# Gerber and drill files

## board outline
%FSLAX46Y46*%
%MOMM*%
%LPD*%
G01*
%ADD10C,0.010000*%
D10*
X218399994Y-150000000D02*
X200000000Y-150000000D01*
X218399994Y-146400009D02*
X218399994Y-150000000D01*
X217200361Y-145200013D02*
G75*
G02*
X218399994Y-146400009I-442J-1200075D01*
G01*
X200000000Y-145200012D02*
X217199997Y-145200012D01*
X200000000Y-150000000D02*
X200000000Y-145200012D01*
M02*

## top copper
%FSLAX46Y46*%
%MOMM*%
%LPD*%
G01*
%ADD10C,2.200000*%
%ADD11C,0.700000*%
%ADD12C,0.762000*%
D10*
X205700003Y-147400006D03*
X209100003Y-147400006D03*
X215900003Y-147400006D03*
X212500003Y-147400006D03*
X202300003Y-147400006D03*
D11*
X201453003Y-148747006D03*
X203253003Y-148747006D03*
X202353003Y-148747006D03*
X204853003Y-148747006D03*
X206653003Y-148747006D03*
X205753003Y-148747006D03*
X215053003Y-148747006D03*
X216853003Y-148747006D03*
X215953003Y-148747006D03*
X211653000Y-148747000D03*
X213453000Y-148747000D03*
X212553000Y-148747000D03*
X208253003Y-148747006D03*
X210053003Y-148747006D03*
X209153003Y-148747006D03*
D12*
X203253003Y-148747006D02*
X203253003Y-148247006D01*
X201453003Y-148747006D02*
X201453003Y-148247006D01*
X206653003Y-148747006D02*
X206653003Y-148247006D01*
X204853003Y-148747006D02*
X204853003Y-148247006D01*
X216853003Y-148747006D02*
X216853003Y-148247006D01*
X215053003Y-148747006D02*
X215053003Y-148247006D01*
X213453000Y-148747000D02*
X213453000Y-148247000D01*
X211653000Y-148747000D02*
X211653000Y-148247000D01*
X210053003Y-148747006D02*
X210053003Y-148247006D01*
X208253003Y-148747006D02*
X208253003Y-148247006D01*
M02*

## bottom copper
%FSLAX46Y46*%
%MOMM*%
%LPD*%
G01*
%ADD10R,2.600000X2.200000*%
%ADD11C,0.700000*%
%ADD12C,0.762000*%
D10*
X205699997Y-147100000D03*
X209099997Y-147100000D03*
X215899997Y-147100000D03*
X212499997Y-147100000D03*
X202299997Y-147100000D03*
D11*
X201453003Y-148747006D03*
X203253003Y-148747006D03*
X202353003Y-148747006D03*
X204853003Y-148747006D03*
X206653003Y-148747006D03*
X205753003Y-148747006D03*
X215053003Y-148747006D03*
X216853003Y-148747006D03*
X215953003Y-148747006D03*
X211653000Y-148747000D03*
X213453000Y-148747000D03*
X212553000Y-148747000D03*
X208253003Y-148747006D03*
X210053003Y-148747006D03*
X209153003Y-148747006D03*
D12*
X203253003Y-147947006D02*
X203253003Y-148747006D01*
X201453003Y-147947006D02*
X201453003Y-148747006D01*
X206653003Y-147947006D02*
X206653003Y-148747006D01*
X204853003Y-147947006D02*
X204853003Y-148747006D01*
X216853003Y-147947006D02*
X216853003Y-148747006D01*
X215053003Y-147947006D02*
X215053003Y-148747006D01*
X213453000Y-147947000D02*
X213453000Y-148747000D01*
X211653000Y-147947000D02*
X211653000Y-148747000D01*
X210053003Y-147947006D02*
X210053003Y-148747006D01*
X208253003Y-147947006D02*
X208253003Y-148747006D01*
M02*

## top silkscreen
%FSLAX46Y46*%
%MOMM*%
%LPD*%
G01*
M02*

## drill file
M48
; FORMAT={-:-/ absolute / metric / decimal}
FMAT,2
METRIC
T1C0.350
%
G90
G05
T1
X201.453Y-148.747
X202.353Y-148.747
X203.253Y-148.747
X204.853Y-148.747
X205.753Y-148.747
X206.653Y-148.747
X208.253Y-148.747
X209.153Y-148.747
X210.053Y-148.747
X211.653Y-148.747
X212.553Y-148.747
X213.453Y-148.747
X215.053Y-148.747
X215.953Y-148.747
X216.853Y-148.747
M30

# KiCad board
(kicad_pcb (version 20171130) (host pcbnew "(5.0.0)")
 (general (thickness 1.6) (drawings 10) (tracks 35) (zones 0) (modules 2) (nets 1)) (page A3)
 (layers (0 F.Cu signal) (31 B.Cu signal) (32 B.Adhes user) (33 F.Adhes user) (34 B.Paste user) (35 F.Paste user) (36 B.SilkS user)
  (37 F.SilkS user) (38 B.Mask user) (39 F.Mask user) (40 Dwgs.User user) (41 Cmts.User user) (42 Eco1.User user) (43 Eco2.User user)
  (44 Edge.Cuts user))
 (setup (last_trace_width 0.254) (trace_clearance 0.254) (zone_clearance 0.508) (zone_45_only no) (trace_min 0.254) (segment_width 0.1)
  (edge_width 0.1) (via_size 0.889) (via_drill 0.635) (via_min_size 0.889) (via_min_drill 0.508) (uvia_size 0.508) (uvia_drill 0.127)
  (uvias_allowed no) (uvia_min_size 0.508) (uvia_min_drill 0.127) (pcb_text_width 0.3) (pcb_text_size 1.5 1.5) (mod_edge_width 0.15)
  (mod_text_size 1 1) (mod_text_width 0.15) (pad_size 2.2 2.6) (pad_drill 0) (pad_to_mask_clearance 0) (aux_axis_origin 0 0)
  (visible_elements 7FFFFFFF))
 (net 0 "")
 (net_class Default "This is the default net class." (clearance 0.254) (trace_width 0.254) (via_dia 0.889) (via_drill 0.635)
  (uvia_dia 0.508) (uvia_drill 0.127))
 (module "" (layer B.Cu) (at 215.800003 147.500006 270)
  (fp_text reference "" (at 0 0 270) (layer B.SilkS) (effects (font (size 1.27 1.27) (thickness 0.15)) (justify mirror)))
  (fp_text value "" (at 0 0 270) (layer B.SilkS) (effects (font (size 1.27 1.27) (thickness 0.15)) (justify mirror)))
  (pad 2 smd circle (at -0.1 10.1 270) (size 2.2 2.2) (layers F.Cu F.Mask))
  (pad 3 smd circle (at -0.1 6.7 270) (size 2.2 2.2) (layers F.Cu F.Mask))
  (pad 5 smd circle (at -0.1 -0.1 270) (size 2.2 2.2) (layers F.Cu F.Mask))
  (pad 4 smd circle (at -0.1 3.3 270) (size 2.2 2.2) (layers F.Cu F.Mask))
  (pad 1 smd circle (at -0.1 13.5 270) (size 2.2 2.2) (layers F.Cu F.Mask)))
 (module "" (layer F.Cu) (at 215.799997 147.800006 90)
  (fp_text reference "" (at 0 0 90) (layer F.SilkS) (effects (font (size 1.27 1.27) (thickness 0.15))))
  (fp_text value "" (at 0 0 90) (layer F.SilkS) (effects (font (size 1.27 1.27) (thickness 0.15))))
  (pad 2 smd rect (at 0.700006 -10.1 90) (size 2.2 2.6) (layers B.Cu B.Mask))
  (pad 3 smd rect (at 0.700006 -6.7 90) (size 2.2 2.6) (layers B.Cu B.Mask))
  (pad 5 smd rect (at 0.700006 0.1 90) (size 2.2 2.6) (layers B.Cu B.Mask))
  (pad 4 smd rect (at 0.700006 -3.3 90) (size 2.2 2.6) (layers B.Cu B.Mask))
  (pad 1 smd rect (at 0.700006 -13.5 90) (size 2.2 2.6) (layers B.Cu B.Mask)))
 (gr_line (start 218.399994 150) (end 200 150) (angle 90) (layer Edge.Cuts) (width 0.01))
 (gr_line (start 218.399994 146.400009) (end 218.399994 150) (angle 90) (layer Edge.Cuts) (width 0.01))
 (gr_arc (start 217.199919 146.400088) (end 218.399994 146.400009) (angle -89.97513145) (layer Edge.Cuts) (width 0.01))
 (gr_line (start 200 145.200012) (end 217.199997 145.200012) (angle 90) (layer Edge.Cuts) (width 0.01))
 (gr_line (start 200 150) (end 200 145.200012) (angle 90) (layer Edge.Cuts) (width 0.01))
 (via (at 201.453003 148.747006) (size 0.7) (drill 0.35) (layers F.Cu B.Cu) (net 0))
 (via (at 203.253003 148.747006) (size 0.7) (drill 0.35) (layers F.Cu B.Cu) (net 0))
 (via (at 202.353003 148.747006) (size 0.7) (drill 0.35) (layers F.Cu B.Cu) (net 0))
 (segment (start 203.253003 147.947006) (end 203.253003 148.747006) (width 0.762) (layer B.Cu) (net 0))
 (segment (start 203.253003 148.747006) (end 203.253003 148.247006) (width 0.762) (layer F.Cu) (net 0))
 (segment (start 201.453003 147.947006) (end 201.453003 148.747006) (width 0.762) (layer B.Cu) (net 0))
 (segment (start 201.453003 148.747006) (end 201.453003 148.247006) (width 0.762) (layer F.Cu) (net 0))
 (via (at 204.853003 148.747006) (size 0.7) (drill 0.35) (layers F.Cu B.Cu) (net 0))
 (via (at 206.653003 148.747006) (size 0.7) (drill 0.35) (layers F.Cu B.Cu) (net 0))
 (via (at 205.753003 148.747006) (size 0.7) (drill 0.35) (layers F.Cu B.Cu) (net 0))
 (segment (start 206.653003 147.947006) (end 206.653003 148.747006) (width 0.762) (layer B.Cu) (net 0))
 (segment (start 206.653003 148.747006) (end 206.653003 148.247006) (width 0.762) (layer F.Cu) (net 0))
 (segment (start 204.853003 147.947006) (end 204.853003 148.747006) (width 0.762) (layer B.Cu) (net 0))
 (segment (start 204.853003 148.747006) (end 204.853003 148.247006) (width 0.762) (layer F.Cu) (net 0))
 (via (at 215.053003 148.747006) (size 0.7) (drill 0.35) (layers F.Cu B.Cu) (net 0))
 (via (at 216.853003 148.747006) (size 0.7) (drill 0.35) (layers F.Cu B.Cu) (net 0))
 (via (at 215.953003 148.747006) (size 0.7) (drill 0.35) (layers F.Cu B.Cu) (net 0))
 (segment (start 216.853003 147.947006) (end 216.853003 148.747006) (width 0.762) (layer B.Cu) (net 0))
 (segment (start 216.853003 148.747006) (end 216.853003 148.247006) (width 0.762) (layer F.Cu) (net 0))
 (segment (start 215.053003 147.947006) (end 215.053003 148.747006) (width 0.762) (layer B.Cu) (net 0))
 (segment (start 215.053003 148.747006) (end 215.053003 148.247006) (width 0.762) (layer F.Cu) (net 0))
 (via (at 211.653 148.747) (size 0.7) (drill 0.35) (layers F.Cu B.Cu) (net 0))
 (via (at 213.453 148.747) (size 0.7) (drill 0.35) (layers F.Cu B.Cu) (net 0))
 (via (at 212.553 148.747) (size 0.7) (drill 0.35) (layers F.Cu B.Cu) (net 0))
 (segment (start 213.453 147.947) (end 213.453 148.747) (width 0.762) (layer B.Cu) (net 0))
 (segment (start 213.453 148.747) (end 213.453 148.247) (width 0.762) (layer F.Cu) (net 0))
 (segment (start 211.653 147.947) (end 211.653 148.747) (width 0.762) (layer B.Cu) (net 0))
 (segment (start 211.653 148.747) (end 211.653 148.247) (width 0.762) (layer F.Cu) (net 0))
 (via (at 208.253003 148.747006) (size 0.7) (drill 0.35) (layers F.Cu B.Cu) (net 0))
 (via (at 210.053003 148.747006) (size 0.7) (drill 0.35) (layers F.Cu B.Cu) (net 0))
 (via (at 209.153003 148.747006) (size 0.7) (drill 0.35) (layers F.Cu B.Cu) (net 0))
 (segment (start 210.053003 147.947006) (end 210.053003 148.747006) (width 0.762) (layer B.Cu) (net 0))
 (segment (start 210.053003 148.747006) (end 210.053003 148.247006) (width 0.762) (layer F.Cu) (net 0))
 (segment (start 208.253003 147.947006) (end 208.253003 148.747006) (width 0.762) (layer B.Cu) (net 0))
 (segment (start 208.253003 148.747006) (end 208.253003 148.247006) (width 0.762) (layer F.Cu) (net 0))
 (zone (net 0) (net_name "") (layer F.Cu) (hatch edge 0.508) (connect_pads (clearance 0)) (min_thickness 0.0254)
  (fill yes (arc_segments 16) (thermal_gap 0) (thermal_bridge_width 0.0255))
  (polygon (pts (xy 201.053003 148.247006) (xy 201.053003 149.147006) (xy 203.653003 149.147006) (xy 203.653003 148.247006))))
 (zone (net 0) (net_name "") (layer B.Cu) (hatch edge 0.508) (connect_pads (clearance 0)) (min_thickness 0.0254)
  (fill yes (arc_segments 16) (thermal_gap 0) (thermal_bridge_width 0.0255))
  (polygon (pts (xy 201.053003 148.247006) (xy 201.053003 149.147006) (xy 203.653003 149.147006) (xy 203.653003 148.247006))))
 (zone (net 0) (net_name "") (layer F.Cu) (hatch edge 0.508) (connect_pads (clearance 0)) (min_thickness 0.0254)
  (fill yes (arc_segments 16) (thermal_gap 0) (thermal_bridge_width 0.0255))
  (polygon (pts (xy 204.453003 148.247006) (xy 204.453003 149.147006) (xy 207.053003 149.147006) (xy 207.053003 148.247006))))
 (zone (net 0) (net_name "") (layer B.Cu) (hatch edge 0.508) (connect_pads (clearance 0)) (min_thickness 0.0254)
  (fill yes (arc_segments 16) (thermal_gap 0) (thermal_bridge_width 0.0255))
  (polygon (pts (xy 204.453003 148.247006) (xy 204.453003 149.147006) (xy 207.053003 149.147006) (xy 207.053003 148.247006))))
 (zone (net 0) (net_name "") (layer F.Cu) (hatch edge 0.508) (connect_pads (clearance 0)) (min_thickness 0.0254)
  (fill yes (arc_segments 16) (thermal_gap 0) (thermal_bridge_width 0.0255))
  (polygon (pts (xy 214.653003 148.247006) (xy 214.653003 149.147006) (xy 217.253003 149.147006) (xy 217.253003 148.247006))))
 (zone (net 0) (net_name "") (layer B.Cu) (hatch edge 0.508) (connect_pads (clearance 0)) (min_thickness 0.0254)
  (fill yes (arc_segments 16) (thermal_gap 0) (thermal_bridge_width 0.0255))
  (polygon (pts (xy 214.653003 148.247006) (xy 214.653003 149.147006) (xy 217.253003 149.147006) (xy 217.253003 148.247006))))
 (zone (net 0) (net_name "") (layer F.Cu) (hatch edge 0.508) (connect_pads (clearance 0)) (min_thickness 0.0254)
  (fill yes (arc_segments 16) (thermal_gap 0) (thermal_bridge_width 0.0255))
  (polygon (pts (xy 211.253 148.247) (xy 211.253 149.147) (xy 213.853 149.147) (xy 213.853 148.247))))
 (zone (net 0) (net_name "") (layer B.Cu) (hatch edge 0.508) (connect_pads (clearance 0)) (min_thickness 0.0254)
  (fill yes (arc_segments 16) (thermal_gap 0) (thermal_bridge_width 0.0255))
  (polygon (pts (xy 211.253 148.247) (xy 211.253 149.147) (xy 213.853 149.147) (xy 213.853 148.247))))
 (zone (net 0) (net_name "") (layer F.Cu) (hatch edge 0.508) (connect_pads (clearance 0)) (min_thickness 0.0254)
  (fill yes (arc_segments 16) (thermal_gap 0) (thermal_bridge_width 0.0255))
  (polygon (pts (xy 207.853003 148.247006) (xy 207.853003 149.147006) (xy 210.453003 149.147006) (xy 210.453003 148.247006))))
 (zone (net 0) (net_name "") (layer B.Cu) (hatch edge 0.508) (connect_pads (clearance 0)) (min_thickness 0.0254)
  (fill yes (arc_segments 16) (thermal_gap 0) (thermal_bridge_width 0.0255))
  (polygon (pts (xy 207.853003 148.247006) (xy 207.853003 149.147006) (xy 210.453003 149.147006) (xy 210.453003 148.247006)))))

